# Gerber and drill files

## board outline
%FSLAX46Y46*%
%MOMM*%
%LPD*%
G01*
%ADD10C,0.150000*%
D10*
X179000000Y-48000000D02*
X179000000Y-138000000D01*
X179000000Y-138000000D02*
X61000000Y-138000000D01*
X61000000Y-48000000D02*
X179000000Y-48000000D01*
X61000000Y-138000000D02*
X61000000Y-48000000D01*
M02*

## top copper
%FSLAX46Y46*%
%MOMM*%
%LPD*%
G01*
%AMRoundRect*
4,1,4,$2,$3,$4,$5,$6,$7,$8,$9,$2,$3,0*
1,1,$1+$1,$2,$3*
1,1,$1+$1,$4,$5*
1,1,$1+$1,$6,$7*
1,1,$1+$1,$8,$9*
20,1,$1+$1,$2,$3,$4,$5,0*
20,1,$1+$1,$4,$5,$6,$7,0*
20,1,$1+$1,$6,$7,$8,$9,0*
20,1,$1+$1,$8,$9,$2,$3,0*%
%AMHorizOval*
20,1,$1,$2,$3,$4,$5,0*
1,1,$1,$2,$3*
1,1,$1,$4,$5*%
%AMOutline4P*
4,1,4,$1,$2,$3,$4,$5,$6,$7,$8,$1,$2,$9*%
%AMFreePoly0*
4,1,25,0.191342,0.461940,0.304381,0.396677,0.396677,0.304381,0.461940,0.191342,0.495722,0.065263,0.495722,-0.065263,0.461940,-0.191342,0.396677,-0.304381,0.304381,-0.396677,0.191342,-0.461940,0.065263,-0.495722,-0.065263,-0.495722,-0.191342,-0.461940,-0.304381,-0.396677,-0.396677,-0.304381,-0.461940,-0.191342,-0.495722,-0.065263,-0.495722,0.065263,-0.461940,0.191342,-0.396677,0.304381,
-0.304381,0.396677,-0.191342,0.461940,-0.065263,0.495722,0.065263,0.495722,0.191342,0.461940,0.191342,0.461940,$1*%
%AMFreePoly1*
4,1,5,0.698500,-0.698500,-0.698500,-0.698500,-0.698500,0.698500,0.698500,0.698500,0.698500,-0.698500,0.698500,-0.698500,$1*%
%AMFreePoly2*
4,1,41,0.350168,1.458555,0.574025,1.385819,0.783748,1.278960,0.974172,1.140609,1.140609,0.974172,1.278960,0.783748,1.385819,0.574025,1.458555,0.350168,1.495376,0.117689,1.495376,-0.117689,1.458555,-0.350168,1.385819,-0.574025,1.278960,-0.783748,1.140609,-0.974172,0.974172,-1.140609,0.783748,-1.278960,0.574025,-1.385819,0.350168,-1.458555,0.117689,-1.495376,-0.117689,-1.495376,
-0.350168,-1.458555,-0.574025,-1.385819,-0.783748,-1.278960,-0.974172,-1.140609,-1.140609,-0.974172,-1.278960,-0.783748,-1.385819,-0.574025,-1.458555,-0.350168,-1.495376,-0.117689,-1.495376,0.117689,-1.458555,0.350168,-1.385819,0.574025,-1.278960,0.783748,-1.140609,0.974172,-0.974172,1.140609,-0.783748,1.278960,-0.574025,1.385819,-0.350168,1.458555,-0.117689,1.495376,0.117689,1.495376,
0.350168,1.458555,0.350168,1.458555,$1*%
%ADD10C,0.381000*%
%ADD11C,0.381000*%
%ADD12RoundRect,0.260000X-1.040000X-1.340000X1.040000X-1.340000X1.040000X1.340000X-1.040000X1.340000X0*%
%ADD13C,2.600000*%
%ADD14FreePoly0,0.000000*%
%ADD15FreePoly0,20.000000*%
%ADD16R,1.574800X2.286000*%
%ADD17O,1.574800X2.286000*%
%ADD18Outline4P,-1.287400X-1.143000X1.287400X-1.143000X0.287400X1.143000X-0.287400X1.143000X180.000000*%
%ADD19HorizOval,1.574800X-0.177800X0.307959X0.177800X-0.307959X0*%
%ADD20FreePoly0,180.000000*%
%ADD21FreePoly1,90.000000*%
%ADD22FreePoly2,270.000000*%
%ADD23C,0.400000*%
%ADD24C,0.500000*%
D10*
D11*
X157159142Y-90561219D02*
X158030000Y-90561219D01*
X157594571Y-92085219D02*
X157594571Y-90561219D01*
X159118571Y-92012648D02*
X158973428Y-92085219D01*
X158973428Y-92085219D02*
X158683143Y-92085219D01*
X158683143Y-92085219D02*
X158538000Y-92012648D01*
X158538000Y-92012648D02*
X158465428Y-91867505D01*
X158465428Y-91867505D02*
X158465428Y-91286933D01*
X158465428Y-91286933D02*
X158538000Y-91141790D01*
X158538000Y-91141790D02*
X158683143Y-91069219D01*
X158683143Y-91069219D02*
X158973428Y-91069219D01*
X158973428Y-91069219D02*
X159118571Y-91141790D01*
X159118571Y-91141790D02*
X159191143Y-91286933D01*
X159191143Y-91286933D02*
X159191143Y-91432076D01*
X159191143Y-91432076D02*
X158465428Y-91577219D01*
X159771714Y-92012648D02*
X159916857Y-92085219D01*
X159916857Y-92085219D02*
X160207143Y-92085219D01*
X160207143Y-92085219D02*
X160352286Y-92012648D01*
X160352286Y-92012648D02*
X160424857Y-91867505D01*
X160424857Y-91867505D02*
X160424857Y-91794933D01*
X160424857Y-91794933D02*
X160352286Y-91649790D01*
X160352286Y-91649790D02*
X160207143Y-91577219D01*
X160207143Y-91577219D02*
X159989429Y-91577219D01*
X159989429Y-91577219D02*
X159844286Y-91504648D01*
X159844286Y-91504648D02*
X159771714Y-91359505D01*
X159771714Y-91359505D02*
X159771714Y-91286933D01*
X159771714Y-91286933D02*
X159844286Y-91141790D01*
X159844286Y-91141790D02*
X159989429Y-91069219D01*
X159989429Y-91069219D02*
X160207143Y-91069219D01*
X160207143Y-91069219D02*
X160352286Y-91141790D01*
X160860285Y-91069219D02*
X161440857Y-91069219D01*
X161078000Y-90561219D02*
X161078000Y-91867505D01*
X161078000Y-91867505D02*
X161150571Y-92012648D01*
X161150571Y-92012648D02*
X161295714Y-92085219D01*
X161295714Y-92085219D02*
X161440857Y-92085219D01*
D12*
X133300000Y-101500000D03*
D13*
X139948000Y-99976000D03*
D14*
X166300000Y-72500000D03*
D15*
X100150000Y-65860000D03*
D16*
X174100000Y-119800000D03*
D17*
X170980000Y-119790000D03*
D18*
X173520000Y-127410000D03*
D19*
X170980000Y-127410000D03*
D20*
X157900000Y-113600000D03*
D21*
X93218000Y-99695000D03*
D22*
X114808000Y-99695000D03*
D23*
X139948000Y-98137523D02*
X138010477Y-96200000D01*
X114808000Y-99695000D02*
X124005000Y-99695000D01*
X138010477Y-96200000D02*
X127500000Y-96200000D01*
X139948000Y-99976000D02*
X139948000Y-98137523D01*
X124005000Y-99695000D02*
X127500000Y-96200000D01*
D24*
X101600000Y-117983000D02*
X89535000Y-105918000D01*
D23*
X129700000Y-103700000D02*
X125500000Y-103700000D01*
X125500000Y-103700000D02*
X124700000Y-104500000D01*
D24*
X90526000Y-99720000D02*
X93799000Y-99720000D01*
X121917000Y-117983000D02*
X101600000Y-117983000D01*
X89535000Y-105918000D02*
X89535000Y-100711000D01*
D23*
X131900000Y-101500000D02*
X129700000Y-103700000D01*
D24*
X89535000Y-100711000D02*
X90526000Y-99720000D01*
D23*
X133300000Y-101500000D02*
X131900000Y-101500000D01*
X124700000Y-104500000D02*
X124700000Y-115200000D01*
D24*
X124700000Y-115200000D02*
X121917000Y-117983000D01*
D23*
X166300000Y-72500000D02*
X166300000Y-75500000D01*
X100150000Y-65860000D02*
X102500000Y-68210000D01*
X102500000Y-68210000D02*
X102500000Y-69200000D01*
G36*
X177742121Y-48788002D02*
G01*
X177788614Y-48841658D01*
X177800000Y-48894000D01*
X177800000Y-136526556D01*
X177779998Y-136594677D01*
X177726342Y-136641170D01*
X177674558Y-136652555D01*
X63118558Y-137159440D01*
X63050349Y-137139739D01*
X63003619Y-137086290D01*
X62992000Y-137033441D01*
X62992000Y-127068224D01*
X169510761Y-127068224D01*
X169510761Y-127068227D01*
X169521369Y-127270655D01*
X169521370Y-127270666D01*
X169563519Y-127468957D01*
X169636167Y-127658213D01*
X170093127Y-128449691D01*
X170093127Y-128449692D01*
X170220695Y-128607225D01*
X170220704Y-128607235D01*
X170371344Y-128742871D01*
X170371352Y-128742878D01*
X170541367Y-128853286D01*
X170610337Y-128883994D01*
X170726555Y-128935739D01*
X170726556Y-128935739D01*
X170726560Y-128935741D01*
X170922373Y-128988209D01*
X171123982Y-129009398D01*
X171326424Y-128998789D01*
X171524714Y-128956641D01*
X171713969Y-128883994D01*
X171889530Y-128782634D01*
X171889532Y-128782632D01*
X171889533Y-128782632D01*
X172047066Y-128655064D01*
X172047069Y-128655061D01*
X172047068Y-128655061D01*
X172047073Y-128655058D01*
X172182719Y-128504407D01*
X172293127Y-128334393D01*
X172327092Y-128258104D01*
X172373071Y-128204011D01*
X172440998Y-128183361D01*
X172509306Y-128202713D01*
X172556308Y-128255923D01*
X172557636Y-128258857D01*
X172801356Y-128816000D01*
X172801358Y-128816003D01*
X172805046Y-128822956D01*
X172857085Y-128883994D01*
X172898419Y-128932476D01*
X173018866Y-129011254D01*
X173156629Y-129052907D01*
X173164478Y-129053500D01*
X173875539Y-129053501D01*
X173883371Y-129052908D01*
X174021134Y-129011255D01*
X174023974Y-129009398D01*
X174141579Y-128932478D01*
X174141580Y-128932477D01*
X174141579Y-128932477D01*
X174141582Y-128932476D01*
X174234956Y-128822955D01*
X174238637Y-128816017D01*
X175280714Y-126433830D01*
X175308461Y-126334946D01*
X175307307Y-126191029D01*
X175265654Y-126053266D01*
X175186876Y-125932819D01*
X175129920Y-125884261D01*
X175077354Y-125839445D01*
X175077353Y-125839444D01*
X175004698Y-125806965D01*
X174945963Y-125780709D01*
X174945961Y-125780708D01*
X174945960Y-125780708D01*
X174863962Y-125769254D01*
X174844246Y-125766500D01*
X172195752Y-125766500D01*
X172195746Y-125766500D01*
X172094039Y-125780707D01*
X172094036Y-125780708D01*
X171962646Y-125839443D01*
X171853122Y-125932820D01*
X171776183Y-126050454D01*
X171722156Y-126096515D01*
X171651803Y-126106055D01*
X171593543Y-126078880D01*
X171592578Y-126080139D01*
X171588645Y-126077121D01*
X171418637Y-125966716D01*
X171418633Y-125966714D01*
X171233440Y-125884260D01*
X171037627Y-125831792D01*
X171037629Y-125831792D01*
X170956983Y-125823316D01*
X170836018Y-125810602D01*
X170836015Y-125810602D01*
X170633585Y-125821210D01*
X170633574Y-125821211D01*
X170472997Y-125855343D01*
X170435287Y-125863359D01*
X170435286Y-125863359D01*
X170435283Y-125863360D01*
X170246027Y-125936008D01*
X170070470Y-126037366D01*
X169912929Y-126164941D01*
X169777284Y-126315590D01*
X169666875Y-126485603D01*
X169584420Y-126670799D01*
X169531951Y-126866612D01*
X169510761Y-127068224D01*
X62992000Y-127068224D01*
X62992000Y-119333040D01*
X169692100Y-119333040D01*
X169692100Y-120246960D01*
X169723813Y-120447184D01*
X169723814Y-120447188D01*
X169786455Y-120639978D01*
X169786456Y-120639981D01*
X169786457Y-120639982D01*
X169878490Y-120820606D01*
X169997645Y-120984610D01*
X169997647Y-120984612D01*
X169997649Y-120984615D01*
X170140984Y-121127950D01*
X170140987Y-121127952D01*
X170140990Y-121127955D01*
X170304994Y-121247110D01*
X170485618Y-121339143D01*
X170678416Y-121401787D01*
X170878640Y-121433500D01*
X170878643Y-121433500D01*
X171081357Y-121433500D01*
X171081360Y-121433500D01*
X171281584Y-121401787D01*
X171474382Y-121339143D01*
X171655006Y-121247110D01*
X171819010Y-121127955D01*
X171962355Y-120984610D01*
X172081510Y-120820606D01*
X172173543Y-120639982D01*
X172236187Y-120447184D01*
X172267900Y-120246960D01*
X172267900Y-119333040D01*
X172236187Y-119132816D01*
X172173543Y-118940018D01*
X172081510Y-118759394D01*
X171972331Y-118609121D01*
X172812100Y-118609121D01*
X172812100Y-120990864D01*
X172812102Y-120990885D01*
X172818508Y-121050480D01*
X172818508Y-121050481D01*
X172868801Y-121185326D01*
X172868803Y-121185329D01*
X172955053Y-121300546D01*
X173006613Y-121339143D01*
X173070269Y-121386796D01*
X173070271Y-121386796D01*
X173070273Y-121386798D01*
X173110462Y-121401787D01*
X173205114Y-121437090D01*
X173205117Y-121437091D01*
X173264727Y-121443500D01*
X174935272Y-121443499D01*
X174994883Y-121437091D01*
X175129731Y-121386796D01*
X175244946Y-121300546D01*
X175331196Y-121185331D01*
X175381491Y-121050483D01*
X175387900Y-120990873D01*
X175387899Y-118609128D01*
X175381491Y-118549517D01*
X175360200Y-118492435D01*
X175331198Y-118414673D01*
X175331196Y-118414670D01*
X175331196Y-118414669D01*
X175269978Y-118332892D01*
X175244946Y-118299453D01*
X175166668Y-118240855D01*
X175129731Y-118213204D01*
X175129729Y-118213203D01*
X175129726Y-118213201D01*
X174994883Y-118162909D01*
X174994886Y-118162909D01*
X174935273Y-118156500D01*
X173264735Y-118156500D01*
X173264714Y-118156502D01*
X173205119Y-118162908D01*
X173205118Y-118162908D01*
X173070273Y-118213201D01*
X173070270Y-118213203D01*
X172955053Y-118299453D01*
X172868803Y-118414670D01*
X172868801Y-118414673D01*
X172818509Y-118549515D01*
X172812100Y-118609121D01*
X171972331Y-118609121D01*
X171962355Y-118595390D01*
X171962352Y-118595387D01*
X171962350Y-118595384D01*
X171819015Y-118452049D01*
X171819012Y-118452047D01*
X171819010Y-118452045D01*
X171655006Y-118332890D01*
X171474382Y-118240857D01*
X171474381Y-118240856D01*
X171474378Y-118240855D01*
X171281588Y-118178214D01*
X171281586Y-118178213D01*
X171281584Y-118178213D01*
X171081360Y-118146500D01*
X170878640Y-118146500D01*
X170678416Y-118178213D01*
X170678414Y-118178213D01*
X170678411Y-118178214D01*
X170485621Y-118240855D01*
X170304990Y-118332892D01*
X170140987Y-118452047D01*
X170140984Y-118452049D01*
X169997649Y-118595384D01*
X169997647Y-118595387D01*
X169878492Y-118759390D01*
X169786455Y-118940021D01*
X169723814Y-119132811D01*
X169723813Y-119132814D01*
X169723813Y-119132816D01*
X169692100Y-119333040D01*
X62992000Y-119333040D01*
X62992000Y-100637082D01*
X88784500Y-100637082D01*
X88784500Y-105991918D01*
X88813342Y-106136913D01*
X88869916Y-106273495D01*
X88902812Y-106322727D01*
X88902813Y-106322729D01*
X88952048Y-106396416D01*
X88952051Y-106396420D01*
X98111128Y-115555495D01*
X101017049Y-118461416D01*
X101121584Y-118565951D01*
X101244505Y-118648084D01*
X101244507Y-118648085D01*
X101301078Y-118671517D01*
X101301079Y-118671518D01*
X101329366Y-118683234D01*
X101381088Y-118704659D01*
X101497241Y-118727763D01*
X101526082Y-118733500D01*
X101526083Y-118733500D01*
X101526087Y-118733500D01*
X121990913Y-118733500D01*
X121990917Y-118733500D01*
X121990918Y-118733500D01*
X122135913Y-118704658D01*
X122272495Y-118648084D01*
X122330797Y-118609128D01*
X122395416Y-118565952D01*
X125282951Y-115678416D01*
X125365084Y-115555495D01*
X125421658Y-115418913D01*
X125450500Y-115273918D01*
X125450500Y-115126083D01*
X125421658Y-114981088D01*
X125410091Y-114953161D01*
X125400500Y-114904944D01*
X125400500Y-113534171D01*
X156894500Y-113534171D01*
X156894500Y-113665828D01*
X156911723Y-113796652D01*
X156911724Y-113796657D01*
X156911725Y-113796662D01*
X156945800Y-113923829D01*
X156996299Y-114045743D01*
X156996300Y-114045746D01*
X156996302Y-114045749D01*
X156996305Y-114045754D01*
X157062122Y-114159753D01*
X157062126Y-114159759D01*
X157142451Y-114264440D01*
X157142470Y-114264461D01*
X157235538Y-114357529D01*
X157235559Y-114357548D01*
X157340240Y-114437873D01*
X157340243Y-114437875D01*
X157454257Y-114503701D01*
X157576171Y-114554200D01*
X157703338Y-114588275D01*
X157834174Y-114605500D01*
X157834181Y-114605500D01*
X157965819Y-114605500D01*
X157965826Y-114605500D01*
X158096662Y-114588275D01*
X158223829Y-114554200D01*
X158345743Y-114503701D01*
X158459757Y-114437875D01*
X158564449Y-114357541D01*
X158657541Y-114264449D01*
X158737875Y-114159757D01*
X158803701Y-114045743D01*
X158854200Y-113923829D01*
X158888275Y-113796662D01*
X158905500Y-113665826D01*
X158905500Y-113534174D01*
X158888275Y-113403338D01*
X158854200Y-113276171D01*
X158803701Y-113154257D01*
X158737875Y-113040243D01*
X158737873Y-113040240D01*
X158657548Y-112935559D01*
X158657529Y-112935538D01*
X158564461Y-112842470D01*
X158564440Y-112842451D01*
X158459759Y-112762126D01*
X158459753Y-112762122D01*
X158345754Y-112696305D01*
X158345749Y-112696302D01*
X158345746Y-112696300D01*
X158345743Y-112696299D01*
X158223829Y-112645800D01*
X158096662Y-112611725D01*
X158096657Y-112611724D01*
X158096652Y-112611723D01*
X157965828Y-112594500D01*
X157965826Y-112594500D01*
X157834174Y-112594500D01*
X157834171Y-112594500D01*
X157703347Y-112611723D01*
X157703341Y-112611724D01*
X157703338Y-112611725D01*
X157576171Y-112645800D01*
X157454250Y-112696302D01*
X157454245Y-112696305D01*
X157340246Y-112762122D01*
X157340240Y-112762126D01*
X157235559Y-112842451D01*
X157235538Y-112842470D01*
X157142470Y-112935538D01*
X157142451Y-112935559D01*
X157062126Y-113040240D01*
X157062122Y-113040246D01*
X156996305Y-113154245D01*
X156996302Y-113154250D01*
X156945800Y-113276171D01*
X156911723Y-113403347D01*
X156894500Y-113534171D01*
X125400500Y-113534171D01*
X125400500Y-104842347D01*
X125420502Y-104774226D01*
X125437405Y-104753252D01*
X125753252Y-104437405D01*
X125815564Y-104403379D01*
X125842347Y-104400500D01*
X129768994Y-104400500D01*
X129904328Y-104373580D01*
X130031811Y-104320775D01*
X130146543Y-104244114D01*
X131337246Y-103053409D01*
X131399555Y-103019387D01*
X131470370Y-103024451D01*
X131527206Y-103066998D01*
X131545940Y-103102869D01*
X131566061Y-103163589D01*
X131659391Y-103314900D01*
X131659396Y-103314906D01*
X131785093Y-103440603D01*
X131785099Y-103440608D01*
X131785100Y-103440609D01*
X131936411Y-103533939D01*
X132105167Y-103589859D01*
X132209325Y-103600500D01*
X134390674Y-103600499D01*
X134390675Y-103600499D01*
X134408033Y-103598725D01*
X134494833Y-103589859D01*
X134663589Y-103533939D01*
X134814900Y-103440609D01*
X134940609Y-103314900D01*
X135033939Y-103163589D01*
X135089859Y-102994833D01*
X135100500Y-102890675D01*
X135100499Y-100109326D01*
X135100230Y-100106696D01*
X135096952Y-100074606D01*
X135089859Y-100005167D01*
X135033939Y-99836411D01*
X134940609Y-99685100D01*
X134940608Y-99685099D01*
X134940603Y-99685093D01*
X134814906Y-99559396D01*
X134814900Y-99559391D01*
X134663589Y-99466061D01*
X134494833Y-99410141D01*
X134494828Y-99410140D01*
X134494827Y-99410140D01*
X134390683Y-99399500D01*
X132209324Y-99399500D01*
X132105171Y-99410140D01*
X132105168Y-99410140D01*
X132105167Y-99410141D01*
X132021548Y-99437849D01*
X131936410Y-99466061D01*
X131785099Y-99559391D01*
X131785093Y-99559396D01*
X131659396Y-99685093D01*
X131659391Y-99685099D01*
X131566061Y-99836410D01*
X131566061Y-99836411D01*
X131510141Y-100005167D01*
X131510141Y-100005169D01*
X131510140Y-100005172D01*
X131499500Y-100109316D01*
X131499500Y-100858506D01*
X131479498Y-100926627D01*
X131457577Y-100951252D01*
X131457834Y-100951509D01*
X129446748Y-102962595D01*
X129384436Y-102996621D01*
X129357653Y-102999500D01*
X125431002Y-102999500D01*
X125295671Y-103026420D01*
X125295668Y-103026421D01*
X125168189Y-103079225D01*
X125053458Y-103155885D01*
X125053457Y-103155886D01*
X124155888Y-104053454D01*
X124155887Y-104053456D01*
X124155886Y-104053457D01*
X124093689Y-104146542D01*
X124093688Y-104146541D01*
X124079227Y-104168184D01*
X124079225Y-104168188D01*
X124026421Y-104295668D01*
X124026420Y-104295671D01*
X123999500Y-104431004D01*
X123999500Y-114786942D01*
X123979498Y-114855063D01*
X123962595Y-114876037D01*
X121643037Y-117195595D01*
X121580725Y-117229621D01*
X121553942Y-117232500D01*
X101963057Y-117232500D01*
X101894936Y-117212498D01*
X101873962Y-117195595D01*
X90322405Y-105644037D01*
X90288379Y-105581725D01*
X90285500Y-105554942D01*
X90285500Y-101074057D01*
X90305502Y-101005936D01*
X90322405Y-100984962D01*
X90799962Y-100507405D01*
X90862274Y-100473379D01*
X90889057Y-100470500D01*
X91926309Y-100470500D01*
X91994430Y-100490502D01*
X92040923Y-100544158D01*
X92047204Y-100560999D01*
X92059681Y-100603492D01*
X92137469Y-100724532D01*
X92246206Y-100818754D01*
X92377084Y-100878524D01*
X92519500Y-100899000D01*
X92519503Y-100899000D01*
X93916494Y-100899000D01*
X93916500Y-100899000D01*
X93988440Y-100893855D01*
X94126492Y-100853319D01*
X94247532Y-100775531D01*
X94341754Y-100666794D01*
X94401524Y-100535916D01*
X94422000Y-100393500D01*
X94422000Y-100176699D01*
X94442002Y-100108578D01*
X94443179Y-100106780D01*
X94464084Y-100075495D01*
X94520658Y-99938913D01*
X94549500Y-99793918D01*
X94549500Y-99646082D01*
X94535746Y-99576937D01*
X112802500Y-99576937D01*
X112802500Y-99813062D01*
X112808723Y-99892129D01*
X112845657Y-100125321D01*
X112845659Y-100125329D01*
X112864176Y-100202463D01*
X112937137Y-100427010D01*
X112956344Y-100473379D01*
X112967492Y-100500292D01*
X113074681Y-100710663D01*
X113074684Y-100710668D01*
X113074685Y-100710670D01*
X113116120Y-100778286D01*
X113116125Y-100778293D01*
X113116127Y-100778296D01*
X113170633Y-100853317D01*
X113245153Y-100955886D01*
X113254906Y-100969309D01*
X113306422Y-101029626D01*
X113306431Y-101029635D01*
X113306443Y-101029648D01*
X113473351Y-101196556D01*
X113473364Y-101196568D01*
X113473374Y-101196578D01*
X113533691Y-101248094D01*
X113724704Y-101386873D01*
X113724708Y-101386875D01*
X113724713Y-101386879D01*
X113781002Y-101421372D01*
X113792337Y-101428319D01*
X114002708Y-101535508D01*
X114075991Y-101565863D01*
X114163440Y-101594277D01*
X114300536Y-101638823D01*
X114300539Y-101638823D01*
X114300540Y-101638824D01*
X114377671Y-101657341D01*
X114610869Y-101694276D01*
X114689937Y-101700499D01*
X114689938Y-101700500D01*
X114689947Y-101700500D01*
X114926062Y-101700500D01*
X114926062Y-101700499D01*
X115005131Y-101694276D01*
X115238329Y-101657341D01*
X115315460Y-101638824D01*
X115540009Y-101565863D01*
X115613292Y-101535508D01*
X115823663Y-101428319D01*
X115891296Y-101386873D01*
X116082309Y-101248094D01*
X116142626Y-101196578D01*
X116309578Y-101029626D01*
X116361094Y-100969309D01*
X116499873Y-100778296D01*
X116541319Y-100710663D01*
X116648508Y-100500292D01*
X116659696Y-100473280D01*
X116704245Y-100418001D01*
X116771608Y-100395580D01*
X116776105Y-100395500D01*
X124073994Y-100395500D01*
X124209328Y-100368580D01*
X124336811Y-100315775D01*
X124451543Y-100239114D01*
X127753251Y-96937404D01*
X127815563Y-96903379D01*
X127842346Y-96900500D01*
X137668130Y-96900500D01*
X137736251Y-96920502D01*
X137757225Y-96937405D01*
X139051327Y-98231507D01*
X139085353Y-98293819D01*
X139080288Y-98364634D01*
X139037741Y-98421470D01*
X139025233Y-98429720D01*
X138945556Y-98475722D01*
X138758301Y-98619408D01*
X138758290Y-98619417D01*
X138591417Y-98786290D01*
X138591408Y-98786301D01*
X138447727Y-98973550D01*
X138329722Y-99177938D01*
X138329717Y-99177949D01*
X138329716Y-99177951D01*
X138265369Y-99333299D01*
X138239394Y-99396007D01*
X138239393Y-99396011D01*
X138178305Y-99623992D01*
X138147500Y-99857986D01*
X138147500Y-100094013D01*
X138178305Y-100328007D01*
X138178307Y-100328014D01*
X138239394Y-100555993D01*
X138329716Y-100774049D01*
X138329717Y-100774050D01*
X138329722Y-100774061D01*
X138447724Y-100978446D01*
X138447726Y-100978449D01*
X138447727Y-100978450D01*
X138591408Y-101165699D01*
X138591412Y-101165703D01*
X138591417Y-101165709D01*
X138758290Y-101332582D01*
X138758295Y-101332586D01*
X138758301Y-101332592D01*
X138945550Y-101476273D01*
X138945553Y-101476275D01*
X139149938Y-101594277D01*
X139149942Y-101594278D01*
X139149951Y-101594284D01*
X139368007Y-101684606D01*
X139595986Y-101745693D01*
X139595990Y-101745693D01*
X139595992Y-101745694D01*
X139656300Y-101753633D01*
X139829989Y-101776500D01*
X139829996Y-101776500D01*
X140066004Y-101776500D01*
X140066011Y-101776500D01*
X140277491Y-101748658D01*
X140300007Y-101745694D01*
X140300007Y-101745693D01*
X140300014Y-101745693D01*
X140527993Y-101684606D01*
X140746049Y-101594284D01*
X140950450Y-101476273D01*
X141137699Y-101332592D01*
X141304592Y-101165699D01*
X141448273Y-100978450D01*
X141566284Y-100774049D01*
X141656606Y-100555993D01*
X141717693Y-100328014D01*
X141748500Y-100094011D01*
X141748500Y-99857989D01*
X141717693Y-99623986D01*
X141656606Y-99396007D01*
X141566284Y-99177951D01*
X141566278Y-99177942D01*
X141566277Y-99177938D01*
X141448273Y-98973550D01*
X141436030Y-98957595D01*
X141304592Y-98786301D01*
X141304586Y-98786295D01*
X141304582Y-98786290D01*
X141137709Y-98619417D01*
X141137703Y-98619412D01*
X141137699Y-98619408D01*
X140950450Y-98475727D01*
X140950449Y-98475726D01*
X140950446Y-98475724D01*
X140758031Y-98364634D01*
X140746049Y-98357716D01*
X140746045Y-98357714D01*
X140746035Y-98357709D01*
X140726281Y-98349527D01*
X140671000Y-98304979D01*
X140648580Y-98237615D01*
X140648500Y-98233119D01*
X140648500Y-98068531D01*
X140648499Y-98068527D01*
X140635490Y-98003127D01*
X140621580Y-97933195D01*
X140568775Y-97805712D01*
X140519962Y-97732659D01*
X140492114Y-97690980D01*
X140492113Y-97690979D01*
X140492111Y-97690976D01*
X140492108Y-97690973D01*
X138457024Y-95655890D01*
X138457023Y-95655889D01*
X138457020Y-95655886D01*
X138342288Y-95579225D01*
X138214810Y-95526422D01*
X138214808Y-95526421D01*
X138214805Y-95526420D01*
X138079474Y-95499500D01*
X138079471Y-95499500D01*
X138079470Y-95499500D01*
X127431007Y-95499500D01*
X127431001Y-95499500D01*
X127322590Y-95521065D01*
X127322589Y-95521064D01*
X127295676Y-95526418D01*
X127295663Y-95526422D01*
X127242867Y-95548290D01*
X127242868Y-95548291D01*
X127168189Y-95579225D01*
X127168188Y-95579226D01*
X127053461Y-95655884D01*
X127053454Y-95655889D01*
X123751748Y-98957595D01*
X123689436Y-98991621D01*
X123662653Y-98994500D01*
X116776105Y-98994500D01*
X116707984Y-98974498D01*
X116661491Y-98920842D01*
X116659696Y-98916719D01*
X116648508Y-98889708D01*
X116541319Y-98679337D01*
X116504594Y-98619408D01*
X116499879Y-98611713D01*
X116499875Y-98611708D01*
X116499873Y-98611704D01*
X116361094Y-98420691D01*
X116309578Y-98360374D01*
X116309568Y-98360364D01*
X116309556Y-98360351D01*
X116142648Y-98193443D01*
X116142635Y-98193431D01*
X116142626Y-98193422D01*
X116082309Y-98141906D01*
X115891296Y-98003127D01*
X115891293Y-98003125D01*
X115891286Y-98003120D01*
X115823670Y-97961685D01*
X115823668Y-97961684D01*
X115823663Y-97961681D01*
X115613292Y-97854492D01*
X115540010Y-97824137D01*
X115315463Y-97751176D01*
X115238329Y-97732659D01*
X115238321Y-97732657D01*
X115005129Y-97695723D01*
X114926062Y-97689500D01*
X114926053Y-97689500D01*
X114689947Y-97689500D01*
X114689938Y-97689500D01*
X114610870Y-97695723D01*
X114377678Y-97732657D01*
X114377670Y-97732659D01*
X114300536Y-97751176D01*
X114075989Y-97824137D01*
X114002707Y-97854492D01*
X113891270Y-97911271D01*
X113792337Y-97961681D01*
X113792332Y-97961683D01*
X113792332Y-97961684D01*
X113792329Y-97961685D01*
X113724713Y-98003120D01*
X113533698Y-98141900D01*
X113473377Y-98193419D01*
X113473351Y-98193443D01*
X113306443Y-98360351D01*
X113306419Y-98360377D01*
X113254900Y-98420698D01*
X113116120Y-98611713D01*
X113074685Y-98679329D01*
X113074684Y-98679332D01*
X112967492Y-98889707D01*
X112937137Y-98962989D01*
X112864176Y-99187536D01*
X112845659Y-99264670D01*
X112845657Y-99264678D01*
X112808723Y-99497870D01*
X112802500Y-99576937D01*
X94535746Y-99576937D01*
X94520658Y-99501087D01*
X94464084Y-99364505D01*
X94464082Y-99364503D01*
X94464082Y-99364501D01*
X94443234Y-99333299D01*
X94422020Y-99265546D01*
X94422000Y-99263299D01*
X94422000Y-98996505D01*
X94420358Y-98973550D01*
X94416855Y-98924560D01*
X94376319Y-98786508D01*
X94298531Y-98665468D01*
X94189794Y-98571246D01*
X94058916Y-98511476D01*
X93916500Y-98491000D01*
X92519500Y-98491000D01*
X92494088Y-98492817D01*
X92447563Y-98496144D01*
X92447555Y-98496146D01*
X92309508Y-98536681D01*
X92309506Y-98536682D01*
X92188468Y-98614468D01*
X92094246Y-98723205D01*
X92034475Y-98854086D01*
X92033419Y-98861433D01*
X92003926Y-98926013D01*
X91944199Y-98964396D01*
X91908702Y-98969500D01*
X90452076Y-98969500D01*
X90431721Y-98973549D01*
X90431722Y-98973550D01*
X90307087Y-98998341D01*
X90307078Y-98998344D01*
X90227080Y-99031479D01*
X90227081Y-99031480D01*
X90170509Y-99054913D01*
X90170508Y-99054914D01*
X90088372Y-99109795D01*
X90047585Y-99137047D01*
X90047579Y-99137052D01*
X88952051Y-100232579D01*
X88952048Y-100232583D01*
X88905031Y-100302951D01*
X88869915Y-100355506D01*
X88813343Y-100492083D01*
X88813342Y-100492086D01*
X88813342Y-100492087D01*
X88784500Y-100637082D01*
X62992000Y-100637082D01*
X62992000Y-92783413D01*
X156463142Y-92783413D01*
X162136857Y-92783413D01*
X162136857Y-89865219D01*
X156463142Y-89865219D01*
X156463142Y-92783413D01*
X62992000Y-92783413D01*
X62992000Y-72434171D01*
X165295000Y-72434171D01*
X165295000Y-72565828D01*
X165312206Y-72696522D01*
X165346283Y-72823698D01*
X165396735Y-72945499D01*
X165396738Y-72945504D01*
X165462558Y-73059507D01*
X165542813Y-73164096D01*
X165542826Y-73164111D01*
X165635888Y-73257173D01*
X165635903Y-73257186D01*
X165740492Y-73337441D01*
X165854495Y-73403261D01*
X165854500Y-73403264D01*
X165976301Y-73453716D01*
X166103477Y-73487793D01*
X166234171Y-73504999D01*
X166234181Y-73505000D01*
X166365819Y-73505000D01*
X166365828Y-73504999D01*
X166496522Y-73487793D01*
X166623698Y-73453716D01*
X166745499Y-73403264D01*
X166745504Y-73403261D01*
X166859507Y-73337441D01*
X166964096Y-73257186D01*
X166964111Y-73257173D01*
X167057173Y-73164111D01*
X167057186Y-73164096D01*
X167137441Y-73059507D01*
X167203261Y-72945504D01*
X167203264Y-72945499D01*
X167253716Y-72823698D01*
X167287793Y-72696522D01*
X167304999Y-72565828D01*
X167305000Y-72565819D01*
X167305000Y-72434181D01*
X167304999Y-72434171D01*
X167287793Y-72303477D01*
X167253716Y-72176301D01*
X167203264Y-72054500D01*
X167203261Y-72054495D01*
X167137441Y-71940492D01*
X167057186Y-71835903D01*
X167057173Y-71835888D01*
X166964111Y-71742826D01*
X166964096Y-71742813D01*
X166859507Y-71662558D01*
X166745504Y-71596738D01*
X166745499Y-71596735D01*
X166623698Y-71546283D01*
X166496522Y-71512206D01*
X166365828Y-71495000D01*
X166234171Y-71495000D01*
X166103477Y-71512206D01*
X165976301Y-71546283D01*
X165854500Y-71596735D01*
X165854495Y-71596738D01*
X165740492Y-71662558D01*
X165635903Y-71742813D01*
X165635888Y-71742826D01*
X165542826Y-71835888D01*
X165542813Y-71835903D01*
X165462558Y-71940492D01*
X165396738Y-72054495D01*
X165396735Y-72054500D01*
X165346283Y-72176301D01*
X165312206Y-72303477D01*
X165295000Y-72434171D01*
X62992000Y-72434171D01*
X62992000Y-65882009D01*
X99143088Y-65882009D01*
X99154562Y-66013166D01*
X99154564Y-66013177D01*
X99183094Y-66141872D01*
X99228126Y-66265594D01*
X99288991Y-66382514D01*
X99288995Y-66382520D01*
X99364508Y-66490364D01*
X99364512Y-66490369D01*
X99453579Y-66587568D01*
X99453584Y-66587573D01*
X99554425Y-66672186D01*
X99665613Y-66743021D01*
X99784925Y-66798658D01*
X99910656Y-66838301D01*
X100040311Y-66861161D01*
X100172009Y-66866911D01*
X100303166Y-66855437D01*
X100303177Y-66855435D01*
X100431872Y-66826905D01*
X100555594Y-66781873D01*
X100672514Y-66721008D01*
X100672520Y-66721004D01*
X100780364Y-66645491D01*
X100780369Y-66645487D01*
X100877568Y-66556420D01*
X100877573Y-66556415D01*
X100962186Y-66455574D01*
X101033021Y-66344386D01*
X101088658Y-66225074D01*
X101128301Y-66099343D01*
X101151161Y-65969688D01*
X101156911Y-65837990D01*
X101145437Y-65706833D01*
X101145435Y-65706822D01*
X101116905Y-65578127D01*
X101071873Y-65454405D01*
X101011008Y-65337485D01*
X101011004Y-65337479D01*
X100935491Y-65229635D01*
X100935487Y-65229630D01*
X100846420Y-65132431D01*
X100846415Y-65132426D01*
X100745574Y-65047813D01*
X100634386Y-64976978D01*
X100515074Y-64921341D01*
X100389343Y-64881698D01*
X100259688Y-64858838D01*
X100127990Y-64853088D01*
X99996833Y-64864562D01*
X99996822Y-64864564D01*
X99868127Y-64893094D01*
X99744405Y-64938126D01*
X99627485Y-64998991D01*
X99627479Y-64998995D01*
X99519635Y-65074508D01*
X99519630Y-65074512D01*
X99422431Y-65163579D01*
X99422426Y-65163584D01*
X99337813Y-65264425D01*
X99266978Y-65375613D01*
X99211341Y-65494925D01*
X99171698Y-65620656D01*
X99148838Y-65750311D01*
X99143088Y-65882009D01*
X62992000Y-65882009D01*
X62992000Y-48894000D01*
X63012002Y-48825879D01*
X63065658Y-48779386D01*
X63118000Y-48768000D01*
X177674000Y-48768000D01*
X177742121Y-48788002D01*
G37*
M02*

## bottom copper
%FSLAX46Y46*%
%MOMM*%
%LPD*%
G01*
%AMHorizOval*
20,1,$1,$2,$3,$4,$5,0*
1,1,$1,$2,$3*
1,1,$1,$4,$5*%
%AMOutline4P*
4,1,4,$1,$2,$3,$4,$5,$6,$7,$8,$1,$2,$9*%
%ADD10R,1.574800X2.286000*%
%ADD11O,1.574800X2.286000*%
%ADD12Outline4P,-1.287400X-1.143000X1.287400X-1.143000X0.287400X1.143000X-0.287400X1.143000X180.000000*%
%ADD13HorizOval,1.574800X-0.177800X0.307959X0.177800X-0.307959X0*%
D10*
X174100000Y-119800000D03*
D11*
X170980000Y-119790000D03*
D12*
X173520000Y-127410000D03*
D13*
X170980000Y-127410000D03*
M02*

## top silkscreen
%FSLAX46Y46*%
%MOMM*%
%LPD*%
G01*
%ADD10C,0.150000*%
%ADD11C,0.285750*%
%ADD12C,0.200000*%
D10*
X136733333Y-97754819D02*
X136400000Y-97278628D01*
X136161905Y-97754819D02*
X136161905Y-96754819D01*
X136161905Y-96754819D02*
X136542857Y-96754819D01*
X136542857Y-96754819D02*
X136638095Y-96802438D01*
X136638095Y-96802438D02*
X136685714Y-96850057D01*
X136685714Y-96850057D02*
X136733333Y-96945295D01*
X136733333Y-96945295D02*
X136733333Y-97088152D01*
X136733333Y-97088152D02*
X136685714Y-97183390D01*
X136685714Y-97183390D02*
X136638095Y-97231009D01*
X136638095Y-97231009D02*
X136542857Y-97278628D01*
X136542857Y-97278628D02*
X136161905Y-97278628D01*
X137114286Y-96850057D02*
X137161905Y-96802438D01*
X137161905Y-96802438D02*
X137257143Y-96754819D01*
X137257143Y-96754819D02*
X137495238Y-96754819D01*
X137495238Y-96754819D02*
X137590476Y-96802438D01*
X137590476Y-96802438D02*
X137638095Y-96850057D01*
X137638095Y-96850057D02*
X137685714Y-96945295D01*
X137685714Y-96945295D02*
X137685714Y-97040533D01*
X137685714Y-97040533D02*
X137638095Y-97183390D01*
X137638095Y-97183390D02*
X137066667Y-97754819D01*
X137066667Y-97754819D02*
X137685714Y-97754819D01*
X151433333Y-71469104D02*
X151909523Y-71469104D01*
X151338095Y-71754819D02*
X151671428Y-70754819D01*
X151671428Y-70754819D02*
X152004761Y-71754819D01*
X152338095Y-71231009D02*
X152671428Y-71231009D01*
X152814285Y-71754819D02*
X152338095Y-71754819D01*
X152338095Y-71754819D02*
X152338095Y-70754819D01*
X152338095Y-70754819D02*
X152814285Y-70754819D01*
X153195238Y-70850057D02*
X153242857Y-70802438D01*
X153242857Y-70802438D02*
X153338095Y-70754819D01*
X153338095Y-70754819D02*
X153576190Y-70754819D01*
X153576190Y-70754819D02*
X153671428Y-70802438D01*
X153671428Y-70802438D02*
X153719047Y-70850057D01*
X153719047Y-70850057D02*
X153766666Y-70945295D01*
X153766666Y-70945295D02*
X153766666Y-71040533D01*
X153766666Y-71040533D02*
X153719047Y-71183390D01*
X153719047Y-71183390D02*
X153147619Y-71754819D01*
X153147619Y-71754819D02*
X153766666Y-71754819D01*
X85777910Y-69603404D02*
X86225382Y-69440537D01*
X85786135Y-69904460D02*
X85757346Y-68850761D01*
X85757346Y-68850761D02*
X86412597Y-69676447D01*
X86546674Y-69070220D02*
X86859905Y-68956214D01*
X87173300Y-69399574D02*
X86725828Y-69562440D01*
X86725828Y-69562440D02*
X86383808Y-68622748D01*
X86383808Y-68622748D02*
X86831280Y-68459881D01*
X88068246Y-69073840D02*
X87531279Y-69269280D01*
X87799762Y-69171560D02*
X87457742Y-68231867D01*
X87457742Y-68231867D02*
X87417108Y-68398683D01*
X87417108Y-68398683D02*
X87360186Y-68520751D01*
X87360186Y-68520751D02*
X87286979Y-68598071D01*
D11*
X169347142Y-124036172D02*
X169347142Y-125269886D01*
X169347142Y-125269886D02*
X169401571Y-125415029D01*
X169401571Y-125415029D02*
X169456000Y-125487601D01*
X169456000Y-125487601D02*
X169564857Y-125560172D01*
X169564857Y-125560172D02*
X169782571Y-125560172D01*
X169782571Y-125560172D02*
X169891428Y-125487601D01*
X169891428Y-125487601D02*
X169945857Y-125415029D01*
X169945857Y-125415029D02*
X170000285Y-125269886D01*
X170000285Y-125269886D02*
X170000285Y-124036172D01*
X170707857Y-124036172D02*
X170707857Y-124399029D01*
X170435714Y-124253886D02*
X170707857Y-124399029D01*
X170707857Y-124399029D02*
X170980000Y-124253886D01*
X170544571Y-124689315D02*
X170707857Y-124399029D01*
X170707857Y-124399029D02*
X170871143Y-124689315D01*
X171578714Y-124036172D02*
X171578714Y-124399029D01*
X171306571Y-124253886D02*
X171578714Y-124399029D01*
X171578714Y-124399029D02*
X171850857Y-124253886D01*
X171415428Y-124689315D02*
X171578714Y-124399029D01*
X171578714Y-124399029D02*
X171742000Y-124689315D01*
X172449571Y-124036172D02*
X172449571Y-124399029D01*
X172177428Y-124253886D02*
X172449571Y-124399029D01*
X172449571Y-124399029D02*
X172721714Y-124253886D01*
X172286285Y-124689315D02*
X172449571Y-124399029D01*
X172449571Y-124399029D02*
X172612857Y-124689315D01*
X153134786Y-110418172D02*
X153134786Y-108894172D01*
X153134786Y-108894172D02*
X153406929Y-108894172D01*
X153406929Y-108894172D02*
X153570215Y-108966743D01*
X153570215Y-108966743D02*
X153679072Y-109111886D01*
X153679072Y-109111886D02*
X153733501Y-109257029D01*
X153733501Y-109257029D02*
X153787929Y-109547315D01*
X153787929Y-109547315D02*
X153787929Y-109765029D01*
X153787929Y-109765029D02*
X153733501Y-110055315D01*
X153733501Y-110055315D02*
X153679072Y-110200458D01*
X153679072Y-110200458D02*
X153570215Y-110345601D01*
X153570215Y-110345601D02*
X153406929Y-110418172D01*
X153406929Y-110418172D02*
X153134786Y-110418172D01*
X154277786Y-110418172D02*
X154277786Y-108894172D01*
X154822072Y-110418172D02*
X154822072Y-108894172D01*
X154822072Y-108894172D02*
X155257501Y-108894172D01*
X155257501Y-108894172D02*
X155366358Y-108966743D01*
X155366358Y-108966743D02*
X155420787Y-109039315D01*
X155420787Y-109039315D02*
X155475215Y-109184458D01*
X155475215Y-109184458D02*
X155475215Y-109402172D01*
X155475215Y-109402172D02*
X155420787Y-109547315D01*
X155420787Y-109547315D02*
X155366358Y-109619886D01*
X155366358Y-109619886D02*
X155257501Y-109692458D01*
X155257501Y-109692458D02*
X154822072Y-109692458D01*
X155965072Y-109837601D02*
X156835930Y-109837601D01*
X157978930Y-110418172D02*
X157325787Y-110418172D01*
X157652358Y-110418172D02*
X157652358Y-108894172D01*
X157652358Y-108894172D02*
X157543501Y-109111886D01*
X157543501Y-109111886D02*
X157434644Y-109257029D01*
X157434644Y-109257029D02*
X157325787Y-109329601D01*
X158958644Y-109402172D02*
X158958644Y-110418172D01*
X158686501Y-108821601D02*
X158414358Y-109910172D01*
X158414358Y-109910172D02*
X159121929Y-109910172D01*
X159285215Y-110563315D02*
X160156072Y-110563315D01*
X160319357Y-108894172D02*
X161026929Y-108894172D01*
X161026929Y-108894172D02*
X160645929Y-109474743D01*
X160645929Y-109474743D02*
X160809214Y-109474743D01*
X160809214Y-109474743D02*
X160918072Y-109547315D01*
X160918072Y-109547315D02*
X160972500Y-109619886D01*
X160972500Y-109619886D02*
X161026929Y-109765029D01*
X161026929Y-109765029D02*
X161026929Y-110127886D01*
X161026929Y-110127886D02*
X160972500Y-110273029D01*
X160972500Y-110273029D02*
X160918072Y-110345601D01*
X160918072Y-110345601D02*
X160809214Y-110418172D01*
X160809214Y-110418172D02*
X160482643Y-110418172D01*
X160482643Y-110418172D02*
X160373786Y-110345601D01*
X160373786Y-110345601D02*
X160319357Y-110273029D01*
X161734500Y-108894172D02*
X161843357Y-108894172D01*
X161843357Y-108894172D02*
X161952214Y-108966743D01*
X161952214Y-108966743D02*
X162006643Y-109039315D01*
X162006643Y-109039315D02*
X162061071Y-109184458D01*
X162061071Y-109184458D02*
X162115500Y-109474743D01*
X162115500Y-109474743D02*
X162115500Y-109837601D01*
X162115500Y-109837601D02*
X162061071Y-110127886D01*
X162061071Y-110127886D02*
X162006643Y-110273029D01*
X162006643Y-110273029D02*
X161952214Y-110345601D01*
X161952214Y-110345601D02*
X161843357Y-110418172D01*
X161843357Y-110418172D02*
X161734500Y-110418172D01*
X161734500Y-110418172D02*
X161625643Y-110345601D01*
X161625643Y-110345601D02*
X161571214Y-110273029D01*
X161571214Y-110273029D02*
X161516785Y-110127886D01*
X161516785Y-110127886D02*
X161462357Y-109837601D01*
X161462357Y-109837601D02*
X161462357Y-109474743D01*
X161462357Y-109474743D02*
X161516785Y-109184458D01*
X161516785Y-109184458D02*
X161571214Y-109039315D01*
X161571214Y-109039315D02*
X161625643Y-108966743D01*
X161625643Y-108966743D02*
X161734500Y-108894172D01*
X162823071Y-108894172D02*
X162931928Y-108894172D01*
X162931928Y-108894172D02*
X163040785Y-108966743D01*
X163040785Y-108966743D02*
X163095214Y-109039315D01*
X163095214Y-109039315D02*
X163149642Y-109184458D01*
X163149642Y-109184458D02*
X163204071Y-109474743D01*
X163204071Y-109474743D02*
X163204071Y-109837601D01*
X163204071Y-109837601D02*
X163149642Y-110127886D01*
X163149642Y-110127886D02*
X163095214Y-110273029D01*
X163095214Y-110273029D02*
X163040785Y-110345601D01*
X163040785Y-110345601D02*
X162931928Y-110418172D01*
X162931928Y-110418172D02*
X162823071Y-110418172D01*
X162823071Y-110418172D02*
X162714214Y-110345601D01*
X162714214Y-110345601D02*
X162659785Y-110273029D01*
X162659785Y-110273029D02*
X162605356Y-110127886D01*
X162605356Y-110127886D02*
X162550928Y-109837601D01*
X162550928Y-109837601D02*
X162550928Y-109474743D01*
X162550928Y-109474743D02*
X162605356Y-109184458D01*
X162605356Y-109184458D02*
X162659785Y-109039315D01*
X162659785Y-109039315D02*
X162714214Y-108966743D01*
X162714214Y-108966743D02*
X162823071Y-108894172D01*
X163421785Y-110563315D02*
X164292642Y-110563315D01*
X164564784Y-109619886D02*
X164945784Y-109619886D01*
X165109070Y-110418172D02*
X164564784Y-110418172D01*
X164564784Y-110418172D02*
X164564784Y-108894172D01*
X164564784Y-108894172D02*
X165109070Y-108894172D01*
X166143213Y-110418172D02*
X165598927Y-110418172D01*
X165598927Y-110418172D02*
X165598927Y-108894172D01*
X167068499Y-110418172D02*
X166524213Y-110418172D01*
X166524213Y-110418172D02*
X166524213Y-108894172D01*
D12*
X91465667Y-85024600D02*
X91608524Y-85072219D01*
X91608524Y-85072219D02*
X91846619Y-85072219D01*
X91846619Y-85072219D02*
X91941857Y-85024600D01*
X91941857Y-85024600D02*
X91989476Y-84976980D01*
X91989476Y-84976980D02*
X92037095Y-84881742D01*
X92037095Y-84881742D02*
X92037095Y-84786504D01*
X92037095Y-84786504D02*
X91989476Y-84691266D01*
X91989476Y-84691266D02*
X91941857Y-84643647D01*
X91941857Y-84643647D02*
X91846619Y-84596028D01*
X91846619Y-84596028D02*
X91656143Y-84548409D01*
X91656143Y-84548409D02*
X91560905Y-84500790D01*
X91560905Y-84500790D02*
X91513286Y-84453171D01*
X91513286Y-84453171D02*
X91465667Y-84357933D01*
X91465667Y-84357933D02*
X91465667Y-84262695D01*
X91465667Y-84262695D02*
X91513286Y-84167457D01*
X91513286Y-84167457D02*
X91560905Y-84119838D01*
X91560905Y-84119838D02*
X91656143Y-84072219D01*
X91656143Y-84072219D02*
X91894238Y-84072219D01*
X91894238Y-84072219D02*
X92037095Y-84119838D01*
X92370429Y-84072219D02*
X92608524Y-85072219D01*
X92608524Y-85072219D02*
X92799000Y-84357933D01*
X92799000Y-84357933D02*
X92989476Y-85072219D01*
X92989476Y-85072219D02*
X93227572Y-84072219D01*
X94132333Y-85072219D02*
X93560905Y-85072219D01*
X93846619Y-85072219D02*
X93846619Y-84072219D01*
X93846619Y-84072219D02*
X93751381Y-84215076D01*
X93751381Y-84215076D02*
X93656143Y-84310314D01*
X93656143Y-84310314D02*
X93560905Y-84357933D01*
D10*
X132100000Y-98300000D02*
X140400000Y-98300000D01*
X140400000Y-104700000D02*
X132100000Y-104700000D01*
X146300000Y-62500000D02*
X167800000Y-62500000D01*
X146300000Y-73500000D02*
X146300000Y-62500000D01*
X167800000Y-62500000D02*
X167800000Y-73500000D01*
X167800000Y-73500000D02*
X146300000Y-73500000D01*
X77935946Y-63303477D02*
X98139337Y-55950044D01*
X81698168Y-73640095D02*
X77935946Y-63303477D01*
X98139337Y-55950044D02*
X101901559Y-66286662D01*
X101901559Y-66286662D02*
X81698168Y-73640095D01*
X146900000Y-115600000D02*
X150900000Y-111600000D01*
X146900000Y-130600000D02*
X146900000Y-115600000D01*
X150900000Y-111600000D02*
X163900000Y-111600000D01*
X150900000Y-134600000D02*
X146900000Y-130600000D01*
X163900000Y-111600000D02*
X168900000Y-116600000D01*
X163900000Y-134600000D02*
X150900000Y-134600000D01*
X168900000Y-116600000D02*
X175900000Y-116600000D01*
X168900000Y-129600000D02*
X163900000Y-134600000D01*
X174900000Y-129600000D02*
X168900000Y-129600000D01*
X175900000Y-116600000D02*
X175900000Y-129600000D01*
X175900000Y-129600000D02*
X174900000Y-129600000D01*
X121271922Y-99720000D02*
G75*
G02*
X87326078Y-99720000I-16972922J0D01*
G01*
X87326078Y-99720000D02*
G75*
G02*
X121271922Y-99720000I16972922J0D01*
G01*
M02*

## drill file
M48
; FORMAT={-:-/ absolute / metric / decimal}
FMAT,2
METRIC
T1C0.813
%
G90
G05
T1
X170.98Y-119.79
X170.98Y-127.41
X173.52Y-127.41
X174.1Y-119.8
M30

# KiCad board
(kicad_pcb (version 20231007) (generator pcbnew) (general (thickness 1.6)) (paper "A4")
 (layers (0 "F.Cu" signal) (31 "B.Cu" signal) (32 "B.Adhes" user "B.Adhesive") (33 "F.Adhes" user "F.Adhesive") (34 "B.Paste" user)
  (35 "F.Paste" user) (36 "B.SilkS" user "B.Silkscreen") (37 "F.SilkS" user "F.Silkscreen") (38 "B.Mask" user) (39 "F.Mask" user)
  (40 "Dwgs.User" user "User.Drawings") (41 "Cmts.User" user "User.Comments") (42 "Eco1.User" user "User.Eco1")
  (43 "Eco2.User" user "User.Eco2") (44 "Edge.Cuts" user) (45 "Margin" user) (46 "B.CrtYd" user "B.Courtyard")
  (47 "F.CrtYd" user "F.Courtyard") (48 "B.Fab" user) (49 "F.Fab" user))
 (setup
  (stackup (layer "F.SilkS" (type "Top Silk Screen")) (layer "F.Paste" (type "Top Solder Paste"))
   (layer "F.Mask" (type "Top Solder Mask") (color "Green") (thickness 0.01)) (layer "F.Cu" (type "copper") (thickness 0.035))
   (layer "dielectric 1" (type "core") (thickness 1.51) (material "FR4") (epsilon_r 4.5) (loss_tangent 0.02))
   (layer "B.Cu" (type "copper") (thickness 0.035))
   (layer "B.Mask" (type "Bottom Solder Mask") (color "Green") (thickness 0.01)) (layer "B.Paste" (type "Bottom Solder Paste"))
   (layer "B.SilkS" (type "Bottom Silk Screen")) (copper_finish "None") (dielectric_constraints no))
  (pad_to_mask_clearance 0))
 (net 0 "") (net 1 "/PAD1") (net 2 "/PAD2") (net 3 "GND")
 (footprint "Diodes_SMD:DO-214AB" (layer "F.Cu") (at 136.9 101.5)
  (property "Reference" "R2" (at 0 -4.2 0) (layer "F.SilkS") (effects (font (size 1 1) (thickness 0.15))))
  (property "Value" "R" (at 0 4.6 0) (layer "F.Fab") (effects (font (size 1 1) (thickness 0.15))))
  (fp_line (start -4.8 -3.2) (end 3.5 -3.2) (stroke (width 0.15) (type solid)) (layer "F.SilkS"))
  (fp_line (start 3.5 3.2) (end -4.8 3.2) (stroke (width 0.15) (type solid)) (layer "F.SilkS"))
  (pad "1" smd roundrect (at -3.6 0) (size 2.6 3.2) (layers "F.Cu" "F.Paste" "F.Mask") (roundrect_rratio 0.1) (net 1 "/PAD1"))
  (pad "2" smd circle (at 3.048 -1.524) (size 2.6 2.6) (layers "F.Cu" "F.Paste" "F.Mask") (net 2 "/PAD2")))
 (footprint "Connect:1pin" (layer "F.Cu") (at 166.3 72.5)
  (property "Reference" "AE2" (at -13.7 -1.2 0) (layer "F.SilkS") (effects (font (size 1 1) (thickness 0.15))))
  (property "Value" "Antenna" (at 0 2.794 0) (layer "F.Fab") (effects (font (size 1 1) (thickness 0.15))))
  (fp_line (start -20 -10) (end 1.5 -10) (stroke (width 0.15) (type solid)) (layer "F.SilkS"))
  (fp_line (start -20 1) (end -20 -10) (stroke (width 0.15) (type solid)) (layer "F.SilkS"))
  (fp_line (start 1.5 -10) (end 1.5 1) (stroke (width 0.15) (type solid)) (layer "F.SilkS"))
  (fp_line (start 1.5 1) (end -20 1) (stroke (width 0.15) (type solid)) (layer "F.SilkS"))
  (pad "1" smd custom (at 0 0) (size 1 1) (layers "F.Cu" "F.Paste" "F.Mask") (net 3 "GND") (zone_connect 0)
   (options (clearance outline) (anchor circle)) (primitives)))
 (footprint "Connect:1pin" (layer "F.Cu") (at 100.15 65.86 20)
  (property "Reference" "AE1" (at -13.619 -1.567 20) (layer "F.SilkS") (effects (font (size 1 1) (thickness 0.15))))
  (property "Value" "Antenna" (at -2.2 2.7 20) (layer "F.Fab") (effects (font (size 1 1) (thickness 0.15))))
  (fp_line (start -20 -10) (end 1.499999 -10) (stroke (width 0.15) (type solid)) (layer "F.SilkS"))
  (fp_line (start -20 1) (end -20 -10) (stroke (width 0.15) (type solid)) (layer "F.SilkS"))
  (fp_line (start 1.499999 -10) (end 1.5 1) (stroke (width 0.15) (type solid)) (layer "F.SilkS"))
  (fp_line (start 1.5 1) (end -20 1) (stroke (width 0.15) (type solid)) (layer "F.SilkS"))
  (pad "1" connect custom (at 0 0 20) (size 1 1) (layers "F.Cu" "F.Mask") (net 3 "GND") (zone_connect 0)
   (options (clearance outline) (anchor circle)) (primitives)))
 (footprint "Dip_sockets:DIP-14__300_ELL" (layer "F.Cu") (at 165.9 123.6 180)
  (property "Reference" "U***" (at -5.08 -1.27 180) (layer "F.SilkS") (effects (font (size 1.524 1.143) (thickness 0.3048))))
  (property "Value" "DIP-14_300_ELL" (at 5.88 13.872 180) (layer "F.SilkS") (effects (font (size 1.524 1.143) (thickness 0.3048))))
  (fp_line (start 19 8) (end 15 12) (stroke (width 0.15) (type solid)) (layer "F.SilkS"))
  (fp_line (start 19 -7) (end 19 8) (stroke (width 0.15) (type solid)) (layer "F.SilkS"))
  (fp_line (start 15 12) (end 2 12) (stroke (width 0.15) (type solid)) (layer "F.SilkS"))
  (fp_line (start 15 -11) (end 19 -7) (stroke (width 0.15) (type solid)) (layer "F.SilkS"))
  (fp_line (start 2 12) (end -3 7) (stroke (width 0.15) (type solid)) (layer "F.SilkS"))
  (fp_line (start 2 -11) (end 15 -11) (stroke (width 0.15) (type solid)) (layer "F.SilkS"))
  (fp_line (start -3 7) (end -10 7) (stroke (width 0.15) (type solid)) (layer "F.SilkS"))
  (fp_line (start -3 -6) (end 2 -11) (stroke (width 0.15) (type solid)) (layer "F.SilkS"))
  (fp_line (start -9 -6) (end -3 -6) (stroke (width 0.15) (type solid)) (layer "F.SilkS"))
  (fp_line (start -10 7) (end -10 -6) (stroke (width 0.15) (type solid)) (layer "F.SilkS"))
  (fp_line (start -10 -6) (end -9 -6) (stroke (width 0.15) (type solid)) (layer "F.SilkS"))
  (pad "1" thru_hole rect (at -8.2 3.8 180) (size 1.5748 2.286) (drill 0.8128) (layers "*.Cu" "*.Mask"))
  (pad "2" thru_hole oval (at -5.08 3.81 180) (size 1.5748 2.286) (drill 0.8128) (layers "*.Cu" "*.Mask"))
  (pad "3" thru_hole trapezoid (at -7.62 -3.81 180) (size 1.5748 2.286) (rect_delta 0 1) (drill 0.8128) (layers "*.Cu" "*.Mask"))
  (pad "4" thru_hole oval (at -5.08 -3.81 210) (size 1.5748 2.286) (drill 0.8128) (layers "*.Cu" "*.Mask"))
  (pad "5" connect custom (at 8 10 180) (size 1 1) (layers "F.Cu" "F.Mask") (zone_connect 0)
   (options (clearance convexhull) (anchor circle)) (primitives)))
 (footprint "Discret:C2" (layer "F.Cu") (at 104.299 99.72)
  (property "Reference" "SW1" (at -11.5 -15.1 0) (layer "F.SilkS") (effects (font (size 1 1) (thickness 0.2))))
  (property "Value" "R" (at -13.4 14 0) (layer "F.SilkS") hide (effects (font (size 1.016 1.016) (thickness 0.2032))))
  (fp_circle (center 0 0) (end 12.065 -11.938) (stroke (width 0.15) (type solid)) (fill none) (layer "F.SilkS"))
  (pad "1" connect custom (at -11.081 -0.025 90) (size 1.397 1.397) (layers "F.Cu" "F.Mask") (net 1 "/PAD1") (solder_mask_margin 0.5)
   (zone_connect 0) (thermal_bridge_angle 45) (options (clearance convexhull) (anchor rect)) (primitives))
  (pad "2" connect custom (at 10.509 -0.025 270) (size 3 3) (layers "F.Cu" "F.Mask") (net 2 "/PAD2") (zone_connect 0)
   (options (clearance outline) (anchor circle)) (primitives)))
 (gr_line (start 179 48) (end 179 138) (stroke (width 0.15) (type solid)) (layer "Edge.Cuts"))
 (gr_line (start 179 138) (end 61 138) (stroke (width 0.15) (type solid)) (layer "Edge.Cuts"))
 (gr_line (start 61 48) (end 179 48) (stroke (width 0.15) (type solid)) (layer "Edge.Cuts"))
 (gr_line (start 61 138) (end 61 48) (stroke (width 0.15) (type solid)) (layer "Edge.Cuts"))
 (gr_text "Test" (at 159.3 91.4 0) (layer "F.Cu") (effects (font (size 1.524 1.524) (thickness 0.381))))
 (segment (start 139.948 98.137523) (end 138.010477 96.2) (width 0.4) (layer "F.Cu") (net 2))
 (segment (start 114.808 99.695) (end 124.005 99.695) (width 0.4) (layer "F.Cu") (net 2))
 (segment (start 138.010477 96.2) (end 127.5 96.2) (width 0.4) (layer "F.Cu") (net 2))
 (segment (start 139.948 99.976) (end 139.948 98.137523) (width 0.4) (layer "F.Cu") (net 2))
 (segment (start 124.005 99.695) (end 127.5 96.2) (width 0.4) (layer "F.Cu") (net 2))
 (segment (start 101.6 117.983) (end 89.535 105.918) (width 0.5) (layer "F.Cu") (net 1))
 (segment (start 129.7 103.7) (end 125.5 103.7) (width 0.4) (layer "F.Cu") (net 1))
 (segment (start 125.5 103.7) (end 124.7 104.5) (width 0.4) (layer "F.Cu") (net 1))
 (segment (start 90.526 99.72) (end 93.799 99.72) (width 0.5) (layer "F.Cu") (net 1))
 (segment (start 121.917 117.983) (end 101.6 117.983) (width 0.5) (layer "F.Cu") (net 1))
 (segment (start 89.535 105.918) (end 89.535 100.711) (width 0.5) (layer "F.Cu") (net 1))
 (segment (start 131.9 101.5) (end 129.7 103.7) (width 0.4) (layer "F.Cu") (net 1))
 (segment (start 89.535 100.711) (end 90.526 99.72) (width 0.5) (layer "F.Cu") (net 1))
 (segment (start 133.3 101.5) (end 131.9 101.5) (width 0.4) (layer "F.Cu") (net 1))
 (segment (start 124.7 104.5) (end 124.7 115.2) (width 0.4) (layer "F.Cu") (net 1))
 (segment (start 124.7 115.2) (end 121.917 117.983) (width 0.5) (layer "F.Cu") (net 1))
 (segment (start 166.3 72.5) (end 166.3 75.5) (width 0.4) (layer "F.Cu") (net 3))
 (segment (start 100.15 65.86) (end 102.5 68.21) (width 0.4) (layer "F.Cu") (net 3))
 (segment (start 102.5 68.21) (end 102.5 69.2) (width 0.4) (layer "F.Cu") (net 3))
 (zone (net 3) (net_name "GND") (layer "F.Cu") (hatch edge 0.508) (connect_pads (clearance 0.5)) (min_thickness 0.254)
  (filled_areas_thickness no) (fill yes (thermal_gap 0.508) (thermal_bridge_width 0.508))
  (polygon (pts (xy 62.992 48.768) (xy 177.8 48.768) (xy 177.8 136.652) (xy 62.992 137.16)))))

